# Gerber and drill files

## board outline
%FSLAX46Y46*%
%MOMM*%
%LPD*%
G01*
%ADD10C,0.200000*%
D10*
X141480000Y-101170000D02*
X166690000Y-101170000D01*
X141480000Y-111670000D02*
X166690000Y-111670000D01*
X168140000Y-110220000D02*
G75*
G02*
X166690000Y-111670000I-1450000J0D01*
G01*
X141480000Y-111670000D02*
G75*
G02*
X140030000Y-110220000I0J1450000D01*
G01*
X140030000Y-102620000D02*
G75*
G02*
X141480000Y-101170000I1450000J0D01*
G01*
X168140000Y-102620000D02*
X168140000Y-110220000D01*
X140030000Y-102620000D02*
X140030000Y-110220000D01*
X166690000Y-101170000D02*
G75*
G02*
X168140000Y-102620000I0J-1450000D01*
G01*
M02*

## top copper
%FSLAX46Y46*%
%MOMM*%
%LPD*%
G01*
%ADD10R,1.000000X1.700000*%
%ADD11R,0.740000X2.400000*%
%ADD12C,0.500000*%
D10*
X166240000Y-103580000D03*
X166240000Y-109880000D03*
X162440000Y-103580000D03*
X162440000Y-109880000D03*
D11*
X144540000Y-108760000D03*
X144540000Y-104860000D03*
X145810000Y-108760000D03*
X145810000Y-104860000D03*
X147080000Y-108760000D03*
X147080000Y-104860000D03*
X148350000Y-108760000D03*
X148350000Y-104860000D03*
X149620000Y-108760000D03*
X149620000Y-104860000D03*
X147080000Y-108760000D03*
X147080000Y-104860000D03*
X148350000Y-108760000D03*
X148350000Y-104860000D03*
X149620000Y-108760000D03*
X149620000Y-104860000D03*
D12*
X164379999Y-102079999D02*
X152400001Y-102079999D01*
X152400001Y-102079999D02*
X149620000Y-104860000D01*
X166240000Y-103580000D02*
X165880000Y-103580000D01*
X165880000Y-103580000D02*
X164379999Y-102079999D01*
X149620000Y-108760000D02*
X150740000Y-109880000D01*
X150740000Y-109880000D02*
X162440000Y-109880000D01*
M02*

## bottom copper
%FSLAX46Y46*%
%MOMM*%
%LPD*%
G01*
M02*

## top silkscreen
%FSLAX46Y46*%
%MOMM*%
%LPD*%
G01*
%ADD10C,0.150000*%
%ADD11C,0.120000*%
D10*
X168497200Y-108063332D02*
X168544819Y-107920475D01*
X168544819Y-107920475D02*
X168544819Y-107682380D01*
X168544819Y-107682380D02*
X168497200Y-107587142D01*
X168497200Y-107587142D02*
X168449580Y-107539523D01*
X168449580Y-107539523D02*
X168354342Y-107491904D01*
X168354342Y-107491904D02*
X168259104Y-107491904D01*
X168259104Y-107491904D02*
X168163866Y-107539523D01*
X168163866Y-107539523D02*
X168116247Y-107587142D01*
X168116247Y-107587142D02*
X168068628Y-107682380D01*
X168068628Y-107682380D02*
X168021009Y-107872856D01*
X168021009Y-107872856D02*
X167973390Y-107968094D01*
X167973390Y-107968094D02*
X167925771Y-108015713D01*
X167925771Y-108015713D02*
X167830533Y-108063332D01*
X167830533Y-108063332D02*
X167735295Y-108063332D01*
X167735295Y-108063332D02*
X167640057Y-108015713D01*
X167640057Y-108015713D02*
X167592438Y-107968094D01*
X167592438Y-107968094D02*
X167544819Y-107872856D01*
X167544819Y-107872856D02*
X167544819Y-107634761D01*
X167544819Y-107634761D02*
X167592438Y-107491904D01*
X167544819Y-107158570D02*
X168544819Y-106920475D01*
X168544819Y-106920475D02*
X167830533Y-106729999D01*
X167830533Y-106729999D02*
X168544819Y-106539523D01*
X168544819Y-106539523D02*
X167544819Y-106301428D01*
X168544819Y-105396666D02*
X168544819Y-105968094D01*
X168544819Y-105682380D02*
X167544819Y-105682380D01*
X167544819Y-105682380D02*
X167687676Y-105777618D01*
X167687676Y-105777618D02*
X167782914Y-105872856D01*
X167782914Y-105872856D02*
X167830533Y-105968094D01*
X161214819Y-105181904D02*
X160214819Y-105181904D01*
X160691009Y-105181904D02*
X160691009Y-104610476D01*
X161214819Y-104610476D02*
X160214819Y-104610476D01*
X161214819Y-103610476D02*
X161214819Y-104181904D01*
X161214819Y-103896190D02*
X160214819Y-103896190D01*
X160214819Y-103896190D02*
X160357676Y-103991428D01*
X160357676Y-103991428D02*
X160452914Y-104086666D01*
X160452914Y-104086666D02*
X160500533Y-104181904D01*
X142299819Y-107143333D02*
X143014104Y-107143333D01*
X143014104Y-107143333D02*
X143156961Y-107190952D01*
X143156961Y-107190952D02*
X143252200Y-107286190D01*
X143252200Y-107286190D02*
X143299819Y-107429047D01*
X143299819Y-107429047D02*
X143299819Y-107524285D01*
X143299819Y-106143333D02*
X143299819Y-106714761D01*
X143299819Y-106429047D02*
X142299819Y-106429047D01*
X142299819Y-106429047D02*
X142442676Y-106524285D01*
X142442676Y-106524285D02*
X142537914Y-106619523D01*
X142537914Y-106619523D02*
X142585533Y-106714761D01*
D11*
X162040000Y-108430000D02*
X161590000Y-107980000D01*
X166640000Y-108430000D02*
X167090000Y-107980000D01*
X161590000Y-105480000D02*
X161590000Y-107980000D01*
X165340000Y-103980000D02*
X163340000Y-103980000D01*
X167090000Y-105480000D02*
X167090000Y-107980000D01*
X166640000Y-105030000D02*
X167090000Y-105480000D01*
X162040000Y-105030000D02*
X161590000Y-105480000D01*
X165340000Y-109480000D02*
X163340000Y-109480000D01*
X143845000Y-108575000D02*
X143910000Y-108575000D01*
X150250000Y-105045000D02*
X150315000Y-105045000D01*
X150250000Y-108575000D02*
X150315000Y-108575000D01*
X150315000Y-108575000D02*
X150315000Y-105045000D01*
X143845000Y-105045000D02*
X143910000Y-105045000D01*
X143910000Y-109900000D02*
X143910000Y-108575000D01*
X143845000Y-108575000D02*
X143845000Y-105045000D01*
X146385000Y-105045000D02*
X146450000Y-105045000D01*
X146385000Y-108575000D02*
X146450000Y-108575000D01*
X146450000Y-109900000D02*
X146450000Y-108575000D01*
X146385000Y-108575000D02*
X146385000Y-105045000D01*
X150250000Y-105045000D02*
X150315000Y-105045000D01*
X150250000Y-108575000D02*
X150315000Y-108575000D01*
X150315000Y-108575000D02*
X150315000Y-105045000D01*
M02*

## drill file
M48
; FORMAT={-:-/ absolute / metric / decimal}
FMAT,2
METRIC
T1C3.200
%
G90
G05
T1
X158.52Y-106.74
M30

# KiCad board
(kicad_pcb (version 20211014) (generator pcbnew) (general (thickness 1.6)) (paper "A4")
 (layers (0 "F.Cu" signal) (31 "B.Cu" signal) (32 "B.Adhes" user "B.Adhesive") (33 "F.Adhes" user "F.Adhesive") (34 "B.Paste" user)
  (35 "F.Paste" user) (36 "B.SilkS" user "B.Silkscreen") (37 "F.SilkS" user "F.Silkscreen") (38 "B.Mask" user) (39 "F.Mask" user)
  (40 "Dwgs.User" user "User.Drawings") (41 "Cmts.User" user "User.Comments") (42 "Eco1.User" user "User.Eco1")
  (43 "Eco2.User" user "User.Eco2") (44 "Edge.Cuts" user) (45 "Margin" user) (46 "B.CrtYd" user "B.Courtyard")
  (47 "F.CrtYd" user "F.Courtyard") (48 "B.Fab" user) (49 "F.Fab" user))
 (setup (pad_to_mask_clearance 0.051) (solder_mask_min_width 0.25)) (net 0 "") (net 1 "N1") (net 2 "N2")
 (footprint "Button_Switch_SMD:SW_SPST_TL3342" (layer "F.Cu") (at 164.34 106.73 -90)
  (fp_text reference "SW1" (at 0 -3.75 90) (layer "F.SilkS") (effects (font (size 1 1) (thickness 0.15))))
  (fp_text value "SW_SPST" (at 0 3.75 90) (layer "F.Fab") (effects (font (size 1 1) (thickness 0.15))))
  (fp_line (start 1.7 2.3) (end 1.25 2.75) (layer "F.SilkS") (width 0.12))
  (fp_line (start 1.7 -2.3) (end 1.25 -2.75) (layer "F.SilkS") (width 0.12))
  (fp_line (start -1.25 2.75) (end 1.25 2.75) (layer "F.SilkS") (width 0.12))
  (fp_line (start -2.75 -1) (end -2.75 1) (layer "F.SilkS") (width 0.12))
  (fp_line (start -1.25 -2.75) (end 1.25 -2.75) (layer "F.SilkS") (width 0.12))
  (fp_line (start -1.7 -2.3) (end -1.25 -2.75) (layer "F.SilkS") (width 0.12))
  (fp_line (start -1.7 2.3) (end -1.25 2.75) (layer "F.SilkS") (width 0.12))
  (fp_line (start 2.75 -1) (end 2.75 1) (layer "F.SilkS") (width 0.12))
  (pad "1" smd rect locked (at -3.15 -1.9 270) (size 1.7 1) (layers "F.Cu" "F.Paste" "F.Mask") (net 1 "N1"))
  (pad "1" smd rect locked (at 3.15 -1.9 270) (size 1.7 1) (layers "F.Cu" "F.Paste" "F.Mask") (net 1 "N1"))
  (pad "2" smd rect locked (at -3.15 1.9 270) (size 1.7 1) (layers "F.Cu" "F.Paste" "F.Mask") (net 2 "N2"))
  (pad "2" smd rect locked (at 3.15 1.9 270) (size 1.7 1) (layers "F.Cu" "F.Paste" "F.Mask") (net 2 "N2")))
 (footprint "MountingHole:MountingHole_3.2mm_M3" (layer "F.Cu") (at 158.38 106.74 -90)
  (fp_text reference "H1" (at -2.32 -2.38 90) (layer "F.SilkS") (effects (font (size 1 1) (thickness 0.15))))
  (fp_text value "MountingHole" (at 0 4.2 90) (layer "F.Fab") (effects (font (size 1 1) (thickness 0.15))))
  (pad "" np_thru_hole circle locked (at 0 -0.14 270) (size 3.2 3.2) (drill 3.2) (layers *.Cu *.Mask)))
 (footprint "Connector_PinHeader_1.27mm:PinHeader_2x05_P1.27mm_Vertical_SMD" (layer "F.Cu") (at 147.08 106.81 90)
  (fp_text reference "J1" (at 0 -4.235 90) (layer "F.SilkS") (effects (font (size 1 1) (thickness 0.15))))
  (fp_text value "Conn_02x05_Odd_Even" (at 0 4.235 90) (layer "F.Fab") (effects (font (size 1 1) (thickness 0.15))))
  (fp_line (start -1.765 -3.235) (end -1.765 -3.17) (layer "F.SilkS") (width 0.12))
  (fp_line (start 1.765 3.17) (end 1.765 3.235) (layer "F.SilkS") (width 0.12))
  (fp_line (start -1.765 3.17) (end -1.765 3.235) (layer "F.SilkS") (width 0.12))
  (fp_line (start -1.765 3.235) (end 1.765 3.235) (layer "F.SilkS") (width 0.12))
  (fp_line (start 1.765 -3.235) (end 1.765 -3.17) (layer "F.SilkS") (width 0.12))
  (fp_line (start -3.09 -3.17) (end -1.765 -3.17) (layer "F.SilkS") (width 0.12))
  (fp_line (start -1.765 -3.235) (end 1.765 -3.235) (layer "F.SilkS") (width 0.12))
  (pad "1" smd rect locked (at -1.95 -2.54 90) (size 2.4 0.74) (layers "F.Cu" "F.Paste" "F.Mask"))
  (pad "2" smd rect locked (at 1.95 -2.54 90) (size 2.4 0.74) (layers "F.Cu" "F.Paste" "F.Mask"))
  (pad "3" smd rect locked (at -1.95 -1.27 90) (size 2.4 0.74) (layers "F.Cu" "F.Paste" "F.Mask"))
  (pad "4" smd rect locked (at 1.95 -1.27 90) (size 2.4 0.74) (layers "F.Cu" "F.Paste" "F.Mask"))
  (pad "5" smd rect locked (at -1.95 0 90) (size 2.4 0.74) (layers "F.Cu" "F.Paste" "F.Mask"))
  (pad "6" smd rect locked (at 1.95 0 90) (size 2.4 0.74) (layers "F.Cu" "F.Paste" "F.Mask"))
  (pad "7" smd rect locked (at -1.95 1.27 90) (size 2.4 0.74) (layers "F.Cu" "F.Paste" "F.Mask"))
  (pad "8" smd rect locked (at 1.95 1.27 90) (size 2.4 0.74) (layers "F.Cu" "F.Paste" "F.Mask"))
  (pad "9" smd rect locked (at -1.95 2.54 90) (size 2.4 0.74) (layers "F.Cu" "F.Paste" "F.Mask") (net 2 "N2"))
  (pad "10" smd rect locked (at 1.95 2.54 90) (size 2.4 0.74) (layers "F.Cu" "F.Paste" "F.Mask") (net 1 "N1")))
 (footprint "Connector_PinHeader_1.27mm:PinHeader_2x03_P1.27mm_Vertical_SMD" (layer "F.Cu") (at 148.35 106.81 90)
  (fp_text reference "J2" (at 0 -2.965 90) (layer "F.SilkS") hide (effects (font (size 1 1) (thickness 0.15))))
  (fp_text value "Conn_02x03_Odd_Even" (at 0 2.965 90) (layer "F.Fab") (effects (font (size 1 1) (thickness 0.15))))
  (fp_line (start 1.765 -1.965) (end 1.765 -1.9) (layer "F.SilkS") (width 0.12))
  (fp_line (start -1.765 -1.965) (end -1.765 -1.9) (layer "F.SilkS") (width 0.12))
  (fp_line (start -3.09 -1.9) (end -1.765 -1.9) (layer "F.SilkS") (width 0.12))
  (fp_line (start -1.765 -1.965) (end 1.765 -1.965) (layer "F.SilkS") (width 0.12))
  (fp_line (start 1.765 1.9) (end 1.765 1.965) (layer "F.SilkS") (width 0.12))
  (fp_line (start -1.765 1.9) (end -1.765 1.965) (layer "F.SilkS") (width 0.12))
  (fp_line (start -1.765 1.965) (end 1.765 1.965) (layer "F.SilkS") (width 0.12))
  (pad "1" smd rect locked (at -1.95 -1.27 90) (size 2.4 0.74) (layers "F.Cu" "F.Paste" "F.Mask"))
  (pad "2" smd rect locked (at 1.95 -1.27 90) (size 2.4 0.74) (layers "F.Cu" "F.Paste" "F.Mask"))
  (pad "3" smd rect locked (at -1.95 0 90) (size 2.4 0.74) (layers "F.Cu" "F.Paste" "F.Mask"))
  (pad "4" smd rect locked (at 1.95 0 90) (size 2.4 0.74) (layers "F.Cu" "F.Paste" "F.Mask"))
  (pad "5" smd rect locked (at -1.95 1.27 90) (size 2.4 0.74) (layers "F.Cu" "F.Paste" "F.Mask") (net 2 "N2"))
  (pad "6" smd rect locked (at 1.95 1.27 90) (size 2.4 0.74) (layers "F.Cu" "F.Paste" "F.Mask") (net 1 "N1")))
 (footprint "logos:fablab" (layer "B.Cu") (at 148.88 102.54)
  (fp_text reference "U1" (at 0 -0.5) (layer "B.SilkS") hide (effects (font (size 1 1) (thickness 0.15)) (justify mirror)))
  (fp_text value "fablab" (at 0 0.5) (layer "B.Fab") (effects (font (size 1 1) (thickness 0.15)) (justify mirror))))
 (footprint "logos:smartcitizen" (layer "B.Cu") (at 164.52 107.1)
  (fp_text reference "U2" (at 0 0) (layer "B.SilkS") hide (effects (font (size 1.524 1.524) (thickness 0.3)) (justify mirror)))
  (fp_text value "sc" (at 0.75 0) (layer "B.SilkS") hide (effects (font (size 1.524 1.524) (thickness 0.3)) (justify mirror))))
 (gr_line (start 141.48 101.17) (end 166.69 101.17) (layer "Edge.Cuts") (width 0.2))
 (gr_line (start 141.48 111.67) (end 166.69 111.67) (layer "Edge.Cuts") (width 0.2))
 (gr_arc (start 168.14 110.22) (mid 167.715305 111.245305) (end 166.69 111.67) (layer "Edge.Cuts") (width 0.2))
 (gr_arc (start 141.48 111.67) (mid 140.454695 111.245305) (end 140.03 110.22) (layer "Edge.Cuts") (width 0.2))
 (gr_arc (start 140.03 102.62) (mid 140.454695 101.594695) (end 141.48 101.17) (layer "Edge.Cuts") (width 0.2))
 (gr_line (start 168.14 102.62) (end 168.14 110.22) (layer "Edge.Cuts") (width 0.2))
 (gr_line (start 140.03 102.62) (end 140.03 110.22) (layer "Edge.Cuts") (width 0.2))
 (gr_arc (start 166.69 101.17) (mid 167.715305 101.594695) (end 168.14 102.62) (layer "Edge.Cuts") (width 0.2))
 (segment (start 164.379999 102.079999) (end 152.400001 102.079999) (width 0.5) (layer "F.Cu") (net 1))
 (segment (start 152.400001 102.079999) (end 149.62 104.86) (width 0.5) (layer "F.Cu") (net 1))
 (segment (start 166.24 103.58) (end 165.88 103.58) (width 0.5) (layer "F.Cu") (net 1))
 (segment (start 165.88 103.58) (end 164.379999 102.079999) (width 0.5) (layer "F.Cu") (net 1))
 (segment (start 149.62 108.76) (end 150.74 109.88) (width 0.5) (layer "F.Cu") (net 2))
 (segment (start 150.74 109.88) (end 162.44 109.88) (width 0.5) (layer "F.Cu") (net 2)))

